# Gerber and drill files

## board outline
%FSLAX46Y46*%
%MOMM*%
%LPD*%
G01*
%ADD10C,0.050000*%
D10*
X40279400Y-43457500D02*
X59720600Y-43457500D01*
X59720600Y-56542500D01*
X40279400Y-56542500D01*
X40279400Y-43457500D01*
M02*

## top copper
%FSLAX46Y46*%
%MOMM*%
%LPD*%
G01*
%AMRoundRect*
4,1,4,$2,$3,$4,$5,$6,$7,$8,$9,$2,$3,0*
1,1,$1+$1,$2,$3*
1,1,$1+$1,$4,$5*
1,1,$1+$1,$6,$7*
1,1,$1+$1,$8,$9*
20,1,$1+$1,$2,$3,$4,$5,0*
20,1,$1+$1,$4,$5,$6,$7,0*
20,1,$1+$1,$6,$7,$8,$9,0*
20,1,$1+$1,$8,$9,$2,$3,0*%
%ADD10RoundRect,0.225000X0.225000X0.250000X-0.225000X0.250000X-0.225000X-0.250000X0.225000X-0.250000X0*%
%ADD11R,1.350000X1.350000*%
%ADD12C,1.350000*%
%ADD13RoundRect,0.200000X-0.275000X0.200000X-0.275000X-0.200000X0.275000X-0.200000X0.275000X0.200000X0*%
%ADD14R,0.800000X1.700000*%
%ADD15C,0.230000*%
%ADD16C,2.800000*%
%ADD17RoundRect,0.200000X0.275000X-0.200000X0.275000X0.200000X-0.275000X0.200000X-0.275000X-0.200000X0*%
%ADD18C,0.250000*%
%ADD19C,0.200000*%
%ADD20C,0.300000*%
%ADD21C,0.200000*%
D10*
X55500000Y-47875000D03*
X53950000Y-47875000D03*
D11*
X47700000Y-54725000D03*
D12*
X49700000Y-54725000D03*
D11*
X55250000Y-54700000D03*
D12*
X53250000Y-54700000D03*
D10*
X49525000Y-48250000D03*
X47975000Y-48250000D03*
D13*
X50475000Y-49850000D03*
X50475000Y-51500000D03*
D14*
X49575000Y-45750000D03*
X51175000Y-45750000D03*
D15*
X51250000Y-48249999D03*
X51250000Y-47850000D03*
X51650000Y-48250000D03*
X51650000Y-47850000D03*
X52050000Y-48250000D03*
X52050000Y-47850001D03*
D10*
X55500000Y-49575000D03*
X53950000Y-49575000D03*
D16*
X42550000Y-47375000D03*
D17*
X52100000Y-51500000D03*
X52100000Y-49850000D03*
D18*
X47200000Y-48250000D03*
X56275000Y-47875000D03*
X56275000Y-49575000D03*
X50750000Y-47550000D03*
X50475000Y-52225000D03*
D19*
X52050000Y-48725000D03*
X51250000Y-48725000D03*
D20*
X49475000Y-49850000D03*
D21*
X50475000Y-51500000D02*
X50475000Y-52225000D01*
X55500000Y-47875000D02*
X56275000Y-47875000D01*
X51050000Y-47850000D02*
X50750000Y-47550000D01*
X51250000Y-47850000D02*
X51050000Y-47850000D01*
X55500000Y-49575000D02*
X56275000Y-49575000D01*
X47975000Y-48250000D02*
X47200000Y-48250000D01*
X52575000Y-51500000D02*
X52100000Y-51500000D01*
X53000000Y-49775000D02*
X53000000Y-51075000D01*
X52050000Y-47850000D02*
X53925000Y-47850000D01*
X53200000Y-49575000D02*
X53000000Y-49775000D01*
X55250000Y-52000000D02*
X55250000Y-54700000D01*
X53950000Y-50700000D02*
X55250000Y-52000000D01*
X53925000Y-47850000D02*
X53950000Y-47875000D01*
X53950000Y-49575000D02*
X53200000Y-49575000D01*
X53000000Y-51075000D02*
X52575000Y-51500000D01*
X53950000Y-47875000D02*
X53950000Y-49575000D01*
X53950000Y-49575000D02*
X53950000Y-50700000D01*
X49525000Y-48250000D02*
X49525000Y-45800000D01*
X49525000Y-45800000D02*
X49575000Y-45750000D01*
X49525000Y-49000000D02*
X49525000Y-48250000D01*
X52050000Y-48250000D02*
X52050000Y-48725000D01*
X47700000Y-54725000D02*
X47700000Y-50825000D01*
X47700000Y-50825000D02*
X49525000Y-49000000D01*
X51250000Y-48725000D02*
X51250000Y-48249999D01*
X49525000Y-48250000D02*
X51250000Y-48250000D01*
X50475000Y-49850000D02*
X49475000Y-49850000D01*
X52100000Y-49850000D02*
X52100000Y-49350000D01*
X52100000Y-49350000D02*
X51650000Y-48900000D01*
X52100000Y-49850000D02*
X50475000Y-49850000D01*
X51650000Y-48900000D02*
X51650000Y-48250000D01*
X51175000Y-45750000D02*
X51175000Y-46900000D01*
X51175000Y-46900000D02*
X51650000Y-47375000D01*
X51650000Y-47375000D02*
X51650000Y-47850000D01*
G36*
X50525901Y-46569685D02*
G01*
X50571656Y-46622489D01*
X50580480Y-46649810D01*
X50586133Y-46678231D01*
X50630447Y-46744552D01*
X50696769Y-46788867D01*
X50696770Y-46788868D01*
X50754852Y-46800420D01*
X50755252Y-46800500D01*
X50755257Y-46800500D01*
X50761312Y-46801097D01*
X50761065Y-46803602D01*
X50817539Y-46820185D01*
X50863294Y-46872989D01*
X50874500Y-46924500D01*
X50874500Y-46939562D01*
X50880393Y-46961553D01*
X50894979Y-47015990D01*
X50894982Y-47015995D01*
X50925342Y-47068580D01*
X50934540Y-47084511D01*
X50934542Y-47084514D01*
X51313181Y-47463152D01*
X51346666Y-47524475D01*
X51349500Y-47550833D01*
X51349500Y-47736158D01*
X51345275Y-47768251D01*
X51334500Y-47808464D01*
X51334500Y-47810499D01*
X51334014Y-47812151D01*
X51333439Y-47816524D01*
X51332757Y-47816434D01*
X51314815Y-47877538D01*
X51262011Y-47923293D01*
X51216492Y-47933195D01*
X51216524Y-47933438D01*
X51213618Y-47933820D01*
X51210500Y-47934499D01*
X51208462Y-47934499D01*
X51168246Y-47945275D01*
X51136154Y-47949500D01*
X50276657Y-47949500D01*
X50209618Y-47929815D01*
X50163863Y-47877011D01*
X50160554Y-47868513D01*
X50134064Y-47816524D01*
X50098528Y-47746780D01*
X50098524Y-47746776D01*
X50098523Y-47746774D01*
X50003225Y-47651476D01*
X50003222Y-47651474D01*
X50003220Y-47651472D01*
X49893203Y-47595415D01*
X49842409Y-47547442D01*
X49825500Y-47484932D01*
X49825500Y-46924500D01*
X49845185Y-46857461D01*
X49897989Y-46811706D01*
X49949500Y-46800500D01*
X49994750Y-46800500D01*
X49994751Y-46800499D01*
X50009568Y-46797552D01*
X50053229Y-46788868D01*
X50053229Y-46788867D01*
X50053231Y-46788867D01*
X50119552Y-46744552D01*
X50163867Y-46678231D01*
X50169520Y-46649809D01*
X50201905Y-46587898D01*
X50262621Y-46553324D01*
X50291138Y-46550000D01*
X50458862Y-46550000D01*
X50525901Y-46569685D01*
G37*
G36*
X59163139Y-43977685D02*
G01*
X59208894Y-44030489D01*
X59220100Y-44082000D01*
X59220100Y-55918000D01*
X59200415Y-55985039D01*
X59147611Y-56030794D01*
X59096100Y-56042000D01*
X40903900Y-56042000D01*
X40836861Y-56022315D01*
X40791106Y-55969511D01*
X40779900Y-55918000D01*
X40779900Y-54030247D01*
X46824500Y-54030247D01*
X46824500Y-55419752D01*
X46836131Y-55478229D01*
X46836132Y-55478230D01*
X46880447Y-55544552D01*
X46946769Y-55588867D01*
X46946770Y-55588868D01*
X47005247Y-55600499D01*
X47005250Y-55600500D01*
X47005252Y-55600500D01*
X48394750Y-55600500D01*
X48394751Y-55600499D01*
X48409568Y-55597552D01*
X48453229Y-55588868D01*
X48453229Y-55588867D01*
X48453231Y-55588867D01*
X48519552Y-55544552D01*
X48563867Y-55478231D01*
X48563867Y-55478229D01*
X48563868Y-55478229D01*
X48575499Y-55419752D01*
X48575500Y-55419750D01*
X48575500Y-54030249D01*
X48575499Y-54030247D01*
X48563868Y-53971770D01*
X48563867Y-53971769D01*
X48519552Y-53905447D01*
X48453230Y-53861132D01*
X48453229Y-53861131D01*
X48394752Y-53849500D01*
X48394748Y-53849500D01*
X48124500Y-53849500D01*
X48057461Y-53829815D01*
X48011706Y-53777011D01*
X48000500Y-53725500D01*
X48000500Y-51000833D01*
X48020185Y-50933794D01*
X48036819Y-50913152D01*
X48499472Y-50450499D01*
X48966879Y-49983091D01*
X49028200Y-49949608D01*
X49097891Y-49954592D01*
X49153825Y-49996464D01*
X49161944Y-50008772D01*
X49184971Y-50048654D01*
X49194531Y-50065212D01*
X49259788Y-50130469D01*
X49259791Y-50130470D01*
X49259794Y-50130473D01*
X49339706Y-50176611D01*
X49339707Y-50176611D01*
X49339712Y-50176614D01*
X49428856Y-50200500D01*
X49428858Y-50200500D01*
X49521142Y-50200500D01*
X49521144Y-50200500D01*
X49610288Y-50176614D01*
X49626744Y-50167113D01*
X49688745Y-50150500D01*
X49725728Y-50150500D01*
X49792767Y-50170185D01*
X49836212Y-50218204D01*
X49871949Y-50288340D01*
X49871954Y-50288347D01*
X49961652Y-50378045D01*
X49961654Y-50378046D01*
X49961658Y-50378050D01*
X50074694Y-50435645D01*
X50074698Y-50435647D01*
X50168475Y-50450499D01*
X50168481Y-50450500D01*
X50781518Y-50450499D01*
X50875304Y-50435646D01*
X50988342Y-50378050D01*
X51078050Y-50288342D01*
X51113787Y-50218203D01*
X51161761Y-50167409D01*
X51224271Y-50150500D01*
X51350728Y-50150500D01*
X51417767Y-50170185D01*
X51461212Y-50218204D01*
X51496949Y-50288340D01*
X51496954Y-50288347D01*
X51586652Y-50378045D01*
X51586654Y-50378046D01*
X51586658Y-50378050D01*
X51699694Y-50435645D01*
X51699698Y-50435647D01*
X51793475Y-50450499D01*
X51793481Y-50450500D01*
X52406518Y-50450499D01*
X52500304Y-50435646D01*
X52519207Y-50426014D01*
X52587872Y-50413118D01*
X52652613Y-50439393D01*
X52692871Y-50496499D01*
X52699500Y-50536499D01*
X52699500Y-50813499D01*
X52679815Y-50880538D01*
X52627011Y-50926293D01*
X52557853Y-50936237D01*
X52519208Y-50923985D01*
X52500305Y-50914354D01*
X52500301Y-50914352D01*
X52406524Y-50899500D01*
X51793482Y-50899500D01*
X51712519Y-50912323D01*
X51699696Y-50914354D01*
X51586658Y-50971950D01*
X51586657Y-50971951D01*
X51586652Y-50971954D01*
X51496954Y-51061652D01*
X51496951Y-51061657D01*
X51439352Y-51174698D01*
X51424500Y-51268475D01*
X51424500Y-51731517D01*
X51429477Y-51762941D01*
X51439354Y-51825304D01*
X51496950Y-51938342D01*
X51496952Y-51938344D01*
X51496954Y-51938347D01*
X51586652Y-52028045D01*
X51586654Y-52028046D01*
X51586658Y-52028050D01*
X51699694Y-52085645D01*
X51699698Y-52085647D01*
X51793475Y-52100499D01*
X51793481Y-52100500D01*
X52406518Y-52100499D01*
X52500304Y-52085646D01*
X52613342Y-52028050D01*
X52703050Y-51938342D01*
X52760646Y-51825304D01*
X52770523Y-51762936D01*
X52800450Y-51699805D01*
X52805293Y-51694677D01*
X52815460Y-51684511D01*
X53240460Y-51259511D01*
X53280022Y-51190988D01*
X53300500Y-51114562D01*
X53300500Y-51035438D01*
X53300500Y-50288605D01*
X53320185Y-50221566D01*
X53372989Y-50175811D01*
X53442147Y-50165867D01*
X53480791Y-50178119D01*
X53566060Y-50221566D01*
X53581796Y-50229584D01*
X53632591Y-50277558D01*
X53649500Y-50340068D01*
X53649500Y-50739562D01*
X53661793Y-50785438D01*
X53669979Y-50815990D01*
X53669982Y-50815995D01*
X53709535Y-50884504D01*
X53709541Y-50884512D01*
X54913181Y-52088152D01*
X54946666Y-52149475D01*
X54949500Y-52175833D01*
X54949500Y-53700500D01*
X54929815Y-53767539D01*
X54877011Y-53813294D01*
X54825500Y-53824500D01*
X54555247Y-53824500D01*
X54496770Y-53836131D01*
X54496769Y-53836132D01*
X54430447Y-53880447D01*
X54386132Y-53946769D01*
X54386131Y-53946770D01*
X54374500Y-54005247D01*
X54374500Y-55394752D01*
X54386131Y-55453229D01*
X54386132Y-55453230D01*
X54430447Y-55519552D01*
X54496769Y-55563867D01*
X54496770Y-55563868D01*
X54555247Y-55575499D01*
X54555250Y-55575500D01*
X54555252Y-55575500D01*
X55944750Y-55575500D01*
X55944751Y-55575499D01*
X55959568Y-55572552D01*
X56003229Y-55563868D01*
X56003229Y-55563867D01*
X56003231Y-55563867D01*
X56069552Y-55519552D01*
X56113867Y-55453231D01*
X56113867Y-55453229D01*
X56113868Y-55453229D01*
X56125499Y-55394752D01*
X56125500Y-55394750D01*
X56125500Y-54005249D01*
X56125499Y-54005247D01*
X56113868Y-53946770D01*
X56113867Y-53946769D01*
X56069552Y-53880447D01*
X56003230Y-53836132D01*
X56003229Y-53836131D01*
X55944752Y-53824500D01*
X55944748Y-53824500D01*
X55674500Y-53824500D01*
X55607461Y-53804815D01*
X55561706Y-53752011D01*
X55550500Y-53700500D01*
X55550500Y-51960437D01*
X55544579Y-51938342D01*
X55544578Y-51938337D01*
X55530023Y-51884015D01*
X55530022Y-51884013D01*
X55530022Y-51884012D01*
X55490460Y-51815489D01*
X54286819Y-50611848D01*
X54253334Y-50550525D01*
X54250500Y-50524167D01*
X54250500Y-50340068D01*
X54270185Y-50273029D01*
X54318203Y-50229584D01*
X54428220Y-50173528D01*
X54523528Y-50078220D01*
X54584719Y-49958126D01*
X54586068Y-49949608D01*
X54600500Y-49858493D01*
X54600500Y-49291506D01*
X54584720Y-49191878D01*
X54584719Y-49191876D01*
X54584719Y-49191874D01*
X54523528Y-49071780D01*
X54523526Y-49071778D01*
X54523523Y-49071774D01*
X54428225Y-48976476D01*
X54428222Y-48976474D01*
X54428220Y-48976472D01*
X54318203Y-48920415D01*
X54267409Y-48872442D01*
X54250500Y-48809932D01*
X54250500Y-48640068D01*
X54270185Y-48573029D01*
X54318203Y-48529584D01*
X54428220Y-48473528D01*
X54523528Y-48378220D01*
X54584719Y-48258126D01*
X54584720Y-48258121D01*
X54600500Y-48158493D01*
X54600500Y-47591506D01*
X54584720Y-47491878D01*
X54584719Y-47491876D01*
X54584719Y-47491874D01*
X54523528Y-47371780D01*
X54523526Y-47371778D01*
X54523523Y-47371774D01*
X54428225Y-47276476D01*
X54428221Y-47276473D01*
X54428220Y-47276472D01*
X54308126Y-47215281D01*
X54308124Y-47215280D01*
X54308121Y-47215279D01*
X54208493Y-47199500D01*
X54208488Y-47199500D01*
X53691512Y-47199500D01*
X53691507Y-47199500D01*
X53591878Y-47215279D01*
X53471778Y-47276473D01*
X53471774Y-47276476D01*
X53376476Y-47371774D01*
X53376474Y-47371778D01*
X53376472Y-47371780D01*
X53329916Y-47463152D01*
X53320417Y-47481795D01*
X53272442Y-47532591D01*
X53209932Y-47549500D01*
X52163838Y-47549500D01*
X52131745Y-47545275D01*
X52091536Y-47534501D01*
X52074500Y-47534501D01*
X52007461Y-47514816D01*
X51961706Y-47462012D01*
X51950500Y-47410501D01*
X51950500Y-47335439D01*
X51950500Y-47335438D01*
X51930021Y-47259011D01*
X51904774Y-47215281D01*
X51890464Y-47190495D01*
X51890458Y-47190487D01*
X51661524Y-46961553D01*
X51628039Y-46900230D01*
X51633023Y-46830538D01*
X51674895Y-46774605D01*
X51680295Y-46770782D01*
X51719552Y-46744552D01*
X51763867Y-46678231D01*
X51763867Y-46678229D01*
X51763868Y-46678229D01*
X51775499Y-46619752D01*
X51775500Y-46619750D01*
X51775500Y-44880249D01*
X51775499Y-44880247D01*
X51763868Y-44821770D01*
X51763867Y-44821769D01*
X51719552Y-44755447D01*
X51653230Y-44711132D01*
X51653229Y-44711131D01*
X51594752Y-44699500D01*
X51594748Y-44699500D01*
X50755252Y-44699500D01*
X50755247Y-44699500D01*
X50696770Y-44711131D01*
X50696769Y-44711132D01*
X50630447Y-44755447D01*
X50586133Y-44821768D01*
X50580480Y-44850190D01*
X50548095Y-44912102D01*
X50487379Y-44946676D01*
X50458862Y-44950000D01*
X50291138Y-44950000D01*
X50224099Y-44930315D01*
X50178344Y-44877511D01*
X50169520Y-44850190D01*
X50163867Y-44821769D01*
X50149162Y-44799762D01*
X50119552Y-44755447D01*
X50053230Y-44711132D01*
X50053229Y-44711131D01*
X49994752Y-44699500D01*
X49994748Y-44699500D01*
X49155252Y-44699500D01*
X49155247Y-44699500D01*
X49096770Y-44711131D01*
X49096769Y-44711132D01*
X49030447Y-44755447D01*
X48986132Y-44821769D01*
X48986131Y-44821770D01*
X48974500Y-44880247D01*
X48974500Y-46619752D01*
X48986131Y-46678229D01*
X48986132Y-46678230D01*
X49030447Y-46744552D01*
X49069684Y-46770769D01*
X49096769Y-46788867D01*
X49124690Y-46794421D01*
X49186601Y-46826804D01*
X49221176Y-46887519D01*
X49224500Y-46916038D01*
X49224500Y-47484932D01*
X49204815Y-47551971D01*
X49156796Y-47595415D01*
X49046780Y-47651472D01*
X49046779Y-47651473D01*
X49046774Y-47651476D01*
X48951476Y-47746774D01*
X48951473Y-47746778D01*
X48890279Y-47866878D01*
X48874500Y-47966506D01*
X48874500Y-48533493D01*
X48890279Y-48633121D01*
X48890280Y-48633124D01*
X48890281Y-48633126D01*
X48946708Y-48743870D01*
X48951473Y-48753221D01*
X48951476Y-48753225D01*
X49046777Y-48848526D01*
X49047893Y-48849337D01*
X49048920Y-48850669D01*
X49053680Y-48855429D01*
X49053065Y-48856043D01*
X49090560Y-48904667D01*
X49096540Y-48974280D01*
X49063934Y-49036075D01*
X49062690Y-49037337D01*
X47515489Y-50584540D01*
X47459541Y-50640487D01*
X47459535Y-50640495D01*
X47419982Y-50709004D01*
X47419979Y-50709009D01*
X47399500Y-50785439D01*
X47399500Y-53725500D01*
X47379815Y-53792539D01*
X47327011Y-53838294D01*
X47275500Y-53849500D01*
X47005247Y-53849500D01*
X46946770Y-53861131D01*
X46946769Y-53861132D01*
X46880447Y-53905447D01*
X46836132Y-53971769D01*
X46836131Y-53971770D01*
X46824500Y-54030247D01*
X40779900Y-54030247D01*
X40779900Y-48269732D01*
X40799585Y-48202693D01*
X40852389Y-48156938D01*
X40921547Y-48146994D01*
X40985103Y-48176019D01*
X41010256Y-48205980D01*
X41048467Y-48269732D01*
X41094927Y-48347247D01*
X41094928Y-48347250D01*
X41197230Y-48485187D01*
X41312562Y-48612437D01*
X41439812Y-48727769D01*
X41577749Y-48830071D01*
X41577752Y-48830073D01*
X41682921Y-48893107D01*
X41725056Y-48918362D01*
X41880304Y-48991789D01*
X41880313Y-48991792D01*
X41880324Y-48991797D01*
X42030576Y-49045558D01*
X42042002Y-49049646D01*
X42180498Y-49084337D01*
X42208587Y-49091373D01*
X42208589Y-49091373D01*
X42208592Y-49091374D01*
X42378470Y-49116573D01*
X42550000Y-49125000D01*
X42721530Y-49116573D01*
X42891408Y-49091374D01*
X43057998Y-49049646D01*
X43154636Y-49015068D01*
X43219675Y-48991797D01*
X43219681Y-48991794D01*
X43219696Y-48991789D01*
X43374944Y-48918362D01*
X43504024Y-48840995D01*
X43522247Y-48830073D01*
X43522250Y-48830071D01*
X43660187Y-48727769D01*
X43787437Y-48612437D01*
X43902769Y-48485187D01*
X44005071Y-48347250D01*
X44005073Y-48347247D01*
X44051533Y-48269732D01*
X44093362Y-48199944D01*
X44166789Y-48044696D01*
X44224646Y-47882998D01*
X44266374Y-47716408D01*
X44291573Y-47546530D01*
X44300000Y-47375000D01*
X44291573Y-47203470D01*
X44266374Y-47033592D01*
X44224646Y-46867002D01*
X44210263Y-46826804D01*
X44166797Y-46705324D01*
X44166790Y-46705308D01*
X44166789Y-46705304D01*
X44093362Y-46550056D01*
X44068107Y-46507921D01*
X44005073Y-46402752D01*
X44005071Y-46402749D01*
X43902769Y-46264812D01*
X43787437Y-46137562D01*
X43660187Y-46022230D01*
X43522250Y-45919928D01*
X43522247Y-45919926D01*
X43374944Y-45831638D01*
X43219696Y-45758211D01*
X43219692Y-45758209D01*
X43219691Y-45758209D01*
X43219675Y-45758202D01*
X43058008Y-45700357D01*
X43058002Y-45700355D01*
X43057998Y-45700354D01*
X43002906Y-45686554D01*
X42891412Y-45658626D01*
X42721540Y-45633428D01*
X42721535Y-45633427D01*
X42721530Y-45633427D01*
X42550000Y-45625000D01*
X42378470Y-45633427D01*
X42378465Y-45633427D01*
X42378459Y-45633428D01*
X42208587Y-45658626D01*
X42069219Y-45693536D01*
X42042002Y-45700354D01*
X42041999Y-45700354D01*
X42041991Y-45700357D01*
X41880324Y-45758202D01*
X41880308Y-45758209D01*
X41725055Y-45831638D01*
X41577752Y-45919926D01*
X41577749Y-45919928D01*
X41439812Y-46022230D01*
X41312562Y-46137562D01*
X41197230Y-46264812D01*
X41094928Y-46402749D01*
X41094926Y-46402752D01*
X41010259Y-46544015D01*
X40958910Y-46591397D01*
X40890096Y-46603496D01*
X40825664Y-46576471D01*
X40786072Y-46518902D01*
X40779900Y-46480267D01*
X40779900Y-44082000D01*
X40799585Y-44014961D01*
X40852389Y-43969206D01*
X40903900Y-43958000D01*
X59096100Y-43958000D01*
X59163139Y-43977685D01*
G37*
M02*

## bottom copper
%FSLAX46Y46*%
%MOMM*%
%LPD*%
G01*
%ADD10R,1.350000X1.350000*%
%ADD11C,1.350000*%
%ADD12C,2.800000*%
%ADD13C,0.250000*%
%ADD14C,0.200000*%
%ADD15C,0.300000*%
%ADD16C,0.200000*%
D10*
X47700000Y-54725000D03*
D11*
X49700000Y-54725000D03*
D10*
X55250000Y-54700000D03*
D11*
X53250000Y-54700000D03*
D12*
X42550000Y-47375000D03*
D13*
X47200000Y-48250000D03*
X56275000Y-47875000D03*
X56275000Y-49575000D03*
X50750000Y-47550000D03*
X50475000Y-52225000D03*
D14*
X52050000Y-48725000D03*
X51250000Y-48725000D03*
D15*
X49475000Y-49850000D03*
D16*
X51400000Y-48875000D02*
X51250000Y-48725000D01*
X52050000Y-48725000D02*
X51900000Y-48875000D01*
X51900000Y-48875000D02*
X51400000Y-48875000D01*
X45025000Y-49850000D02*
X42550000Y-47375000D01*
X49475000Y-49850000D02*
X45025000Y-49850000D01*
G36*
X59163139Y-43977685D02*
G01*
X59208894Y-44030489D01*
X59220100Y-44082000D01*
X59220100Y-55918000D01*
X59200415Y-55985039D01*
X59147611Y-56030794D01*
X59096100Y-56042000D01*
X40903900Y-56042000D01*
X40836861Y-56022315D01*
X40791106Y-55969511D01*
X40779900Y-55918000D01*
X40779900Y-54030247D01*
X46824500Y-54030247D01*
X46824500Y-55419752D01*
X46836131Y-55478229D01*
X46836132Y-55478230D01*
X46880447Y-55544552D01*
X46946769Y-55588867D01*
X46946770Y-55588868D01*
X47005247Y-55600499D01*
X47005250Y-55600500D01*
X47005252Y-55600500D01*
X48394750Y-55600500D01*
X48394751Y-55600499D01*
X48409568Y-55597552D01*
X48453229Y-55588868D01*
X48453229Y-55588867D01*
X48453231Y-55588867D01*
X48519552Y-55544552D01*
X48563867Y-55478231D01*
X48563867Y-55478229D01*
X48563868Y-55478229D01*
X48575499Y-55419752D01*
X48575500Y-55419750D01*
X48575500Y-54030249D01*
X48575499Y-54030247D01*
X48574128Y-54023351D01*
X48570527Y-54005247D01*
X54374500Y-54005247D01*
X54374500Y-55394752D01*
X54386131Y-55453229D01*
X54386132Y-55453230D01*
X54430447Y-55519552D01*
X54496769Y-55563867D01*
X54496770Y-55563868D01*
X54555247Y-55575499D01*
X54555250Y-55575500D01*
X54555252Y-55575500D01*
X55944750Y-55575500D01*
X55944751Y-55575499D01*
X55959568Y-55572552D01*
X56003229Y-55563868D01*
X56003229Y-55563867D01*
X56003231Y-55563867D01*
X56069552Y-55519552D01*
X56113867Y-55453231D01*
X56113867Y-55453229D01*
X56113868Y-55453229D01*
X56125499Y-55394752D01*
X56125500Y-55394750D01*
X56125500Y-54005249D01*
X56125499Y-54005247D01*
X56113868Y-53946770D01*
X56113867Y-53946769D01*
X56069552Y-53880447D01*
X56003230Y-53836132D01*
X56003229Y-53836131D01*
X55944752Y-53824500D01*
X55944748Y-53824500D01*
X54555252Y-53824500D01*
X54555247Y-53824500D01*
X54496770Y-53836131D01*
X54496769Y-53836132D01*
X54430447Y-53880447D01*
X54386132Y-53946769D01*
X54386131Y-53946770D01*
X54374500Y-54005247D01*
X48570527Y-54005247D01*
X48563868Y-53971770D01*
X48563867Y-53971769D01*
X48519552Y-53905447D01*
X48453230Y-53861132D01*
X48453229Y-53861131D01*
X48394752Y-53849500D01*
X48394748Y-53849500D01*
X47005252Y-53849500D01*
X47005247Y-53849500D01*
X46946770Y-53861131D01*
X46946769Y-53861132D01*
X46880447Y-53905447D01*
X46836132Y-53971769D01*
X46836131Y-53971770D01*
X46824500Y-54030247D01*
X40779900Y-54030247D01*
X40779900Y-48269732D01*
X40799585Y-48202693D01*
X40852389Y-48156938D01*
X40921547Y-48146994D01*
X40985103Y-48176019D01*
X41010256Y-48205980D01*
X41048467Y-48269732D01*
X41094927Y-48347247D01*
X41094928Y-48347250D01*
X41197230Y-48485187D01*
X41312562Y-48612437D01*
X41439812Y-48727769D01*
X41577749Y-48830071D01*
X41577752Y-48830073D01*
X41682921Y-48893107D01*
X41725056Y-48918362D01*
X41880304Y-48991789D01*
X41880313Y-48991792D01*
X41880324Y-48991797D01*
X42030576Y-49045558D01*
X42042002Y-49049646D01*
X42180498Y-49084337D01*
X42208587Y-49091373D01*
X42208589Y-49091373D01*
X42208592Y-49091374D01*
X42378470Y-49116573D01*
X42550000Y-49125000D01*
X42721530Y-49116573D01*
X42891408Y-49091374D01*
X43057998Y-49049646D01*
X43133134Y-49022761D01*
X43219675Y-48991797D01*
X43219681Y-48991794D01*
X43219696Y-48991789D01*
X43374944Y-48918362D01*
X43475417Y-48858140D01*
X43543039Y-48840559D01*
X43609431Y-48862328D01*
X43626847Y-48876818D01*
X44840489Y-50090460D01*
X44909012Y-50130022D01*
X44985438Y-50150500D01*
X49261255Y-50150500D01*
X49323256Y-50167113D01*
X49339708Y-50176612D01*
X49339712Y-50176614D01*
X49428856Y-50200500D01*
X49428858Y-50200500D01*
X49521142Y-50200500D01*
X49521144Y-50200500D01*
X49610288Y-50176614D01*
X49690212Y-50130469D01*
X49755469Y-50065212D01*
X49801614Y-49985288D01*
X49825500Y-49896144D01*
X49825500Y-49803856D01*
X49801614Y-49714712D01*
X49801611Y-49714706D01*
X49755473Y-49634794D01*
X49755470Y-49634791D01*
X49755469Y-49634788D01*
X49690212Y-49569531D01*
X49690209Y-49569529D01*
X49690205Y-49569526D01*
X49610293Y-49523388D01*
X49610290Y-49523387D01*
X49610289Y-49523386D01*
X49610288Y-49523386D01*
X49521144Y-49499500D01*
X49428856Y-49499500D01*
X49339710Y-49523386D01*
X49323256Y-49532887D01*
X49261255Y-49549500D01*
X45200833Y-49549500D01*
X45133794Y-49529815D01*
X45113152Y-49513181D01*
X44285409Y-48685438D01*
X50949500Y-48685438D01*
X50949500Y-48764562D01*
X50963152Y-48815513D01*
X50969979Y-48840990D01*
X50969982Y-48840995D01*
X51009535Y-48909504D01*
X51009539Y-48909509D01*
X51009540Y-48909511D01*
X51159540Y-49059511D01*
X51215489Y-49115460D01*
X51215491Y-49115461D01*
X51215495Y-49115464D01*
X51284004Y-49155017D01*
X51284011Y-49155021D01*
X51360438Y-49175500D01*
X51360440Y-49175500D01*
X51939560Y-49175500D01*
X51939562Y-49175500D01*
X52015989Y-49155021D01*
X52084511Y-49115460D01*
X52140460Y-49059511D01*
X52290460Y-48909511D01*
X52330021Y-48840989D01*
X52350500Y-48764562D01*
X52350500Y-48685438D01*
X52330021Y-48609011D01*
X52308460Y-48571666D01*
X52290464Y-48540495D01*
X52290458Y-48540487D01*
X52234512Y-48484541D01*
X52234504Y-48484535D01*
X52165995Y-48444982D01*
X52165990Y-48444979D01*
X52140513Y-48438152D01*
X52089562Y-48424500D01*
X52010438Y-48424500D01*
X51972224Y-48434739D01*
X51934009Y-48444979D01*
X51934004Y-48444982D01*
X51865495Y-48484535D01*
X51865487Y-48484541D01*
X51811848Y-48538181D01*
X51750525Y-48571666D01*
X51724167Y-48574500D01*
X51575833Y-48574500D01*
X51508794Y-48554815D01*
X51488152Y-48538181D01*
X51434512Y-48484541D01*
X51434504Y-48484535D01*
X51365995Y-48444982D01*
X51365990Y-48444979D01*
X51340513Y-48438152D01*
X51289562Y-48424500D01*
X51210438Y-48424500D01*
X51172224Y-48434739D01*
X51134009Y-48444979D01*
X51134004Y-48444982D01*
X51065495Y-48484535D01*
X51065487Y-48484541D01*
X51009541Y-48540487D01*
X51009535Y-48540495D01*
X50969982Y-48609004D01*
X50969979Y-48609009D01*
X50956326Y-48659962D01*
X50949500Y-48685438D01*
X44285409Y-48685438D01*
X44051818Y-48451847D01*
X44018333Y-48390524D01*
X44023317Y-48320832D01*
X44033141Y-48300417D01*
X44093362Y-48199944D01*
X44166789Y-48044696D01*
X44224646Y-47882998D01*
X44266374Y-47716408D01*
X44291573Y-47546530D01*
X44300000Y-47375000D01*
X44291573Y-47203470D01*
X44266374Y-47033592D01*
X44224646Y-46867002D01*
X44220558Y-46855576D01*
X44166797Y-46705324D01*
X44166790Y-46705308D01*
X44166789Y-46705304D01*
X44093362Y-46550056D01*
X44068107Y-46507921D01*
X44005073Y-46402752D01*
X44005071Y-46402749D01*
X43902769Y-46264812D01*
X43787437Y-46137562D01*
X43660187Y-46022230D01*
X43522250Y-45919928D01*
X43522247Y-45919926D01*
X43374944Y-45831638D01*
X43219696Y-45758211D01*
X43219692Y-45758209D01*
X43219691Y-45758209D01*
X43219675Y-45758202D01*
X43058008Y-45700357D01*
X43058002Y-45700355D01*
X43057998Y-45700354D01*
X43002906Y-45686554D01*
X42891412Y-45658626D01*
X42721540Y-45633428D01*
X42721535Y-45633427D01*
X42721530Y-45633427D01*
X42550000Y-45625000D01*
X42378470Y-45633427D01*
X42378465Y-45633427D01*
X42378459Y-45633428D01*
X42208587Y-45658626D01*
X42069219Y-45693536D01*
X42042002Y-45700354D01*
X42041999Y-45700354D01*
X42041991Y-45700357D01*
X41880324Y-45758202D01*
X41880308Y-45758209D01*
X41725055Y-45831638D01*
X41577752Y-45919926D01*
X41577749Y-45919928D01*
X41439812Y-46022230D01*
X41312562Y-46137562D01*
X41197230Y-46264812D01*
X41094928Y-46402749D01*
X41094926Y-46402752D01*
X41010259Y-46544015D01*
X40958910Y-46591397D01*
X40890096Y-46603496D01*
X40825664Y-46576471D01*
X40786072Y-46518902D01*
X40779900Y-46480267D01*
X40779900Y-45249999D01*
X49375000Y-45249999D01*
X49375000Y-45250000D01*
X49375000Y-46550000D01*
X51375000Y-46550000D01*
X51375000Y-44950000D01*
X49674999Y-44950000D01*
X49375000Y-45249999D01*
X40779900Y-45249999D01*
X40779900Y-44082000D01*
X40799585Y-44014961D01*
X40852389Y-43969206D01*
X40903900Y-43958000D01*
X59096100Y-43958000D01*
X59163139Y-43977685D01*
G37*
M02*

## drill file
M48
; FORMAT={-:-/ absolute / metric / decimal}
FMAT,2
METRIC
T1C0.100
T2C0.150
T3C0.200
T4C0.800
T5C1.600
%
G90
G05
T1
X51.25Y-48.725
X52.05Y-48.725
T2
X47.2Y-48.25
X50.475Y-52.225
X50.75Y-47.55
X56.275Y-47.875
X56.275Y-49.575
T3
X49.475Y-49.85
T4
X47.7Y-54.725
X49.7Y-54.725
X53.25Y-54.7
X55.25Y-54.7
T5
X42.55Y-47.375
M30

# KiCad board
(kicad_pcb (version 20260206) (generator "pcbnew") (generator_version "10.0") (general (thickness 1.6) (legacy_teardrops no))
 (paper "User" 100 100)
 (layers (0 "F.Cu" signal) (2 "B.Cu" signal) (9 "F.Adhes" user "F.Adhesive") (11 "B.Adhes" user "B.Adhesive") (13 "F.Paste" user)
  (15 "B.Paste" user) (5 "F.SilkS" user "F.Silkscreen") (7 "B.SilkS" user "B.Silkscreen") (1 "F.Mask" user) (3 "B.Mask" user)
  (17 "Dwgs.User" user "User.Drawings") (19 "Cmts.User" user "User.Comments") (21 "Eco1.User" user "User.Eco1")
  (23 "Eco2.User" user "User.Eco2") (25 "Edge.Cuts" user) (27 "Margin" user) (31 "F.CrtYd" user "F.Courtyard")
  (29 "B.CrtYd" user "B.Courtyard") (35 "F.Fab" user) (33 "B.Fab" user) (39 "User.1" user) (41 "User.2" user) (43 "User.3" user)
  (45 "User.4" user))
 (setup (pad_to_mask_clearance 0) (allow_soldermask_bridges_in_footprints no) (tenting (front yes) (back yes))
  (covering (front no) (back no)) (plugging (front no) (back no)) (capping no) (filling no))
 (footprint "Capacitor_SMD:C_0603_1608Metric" (layer "F.Cu") (at 54.725 47.875 180)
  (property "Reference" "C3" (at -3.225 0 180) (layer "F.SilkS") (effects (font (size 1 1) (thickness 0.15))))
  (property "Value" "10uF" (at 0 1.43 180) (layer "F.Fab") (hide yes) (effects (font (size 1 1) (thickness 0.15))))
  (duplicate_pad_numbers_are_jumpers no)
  (pad "1" smd roundrect (at -0.775 0 180) (size 0.9 0.95) (layers "F.Cu" "F.Mask" "F.Paste") (roundrect_rratio 0.25) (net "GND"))
  (pad "2" smd roundrect (at 0.775 0 180) (size 0.9 0.95) (layers "F.Cu" "F.Mask" "F.Paste") (roundrect_rratio 0.25) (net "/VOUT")))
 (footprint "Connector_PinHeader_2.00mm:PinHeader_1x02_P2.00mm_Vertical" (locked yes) (layer "F.Cu") (at 48.7 54.725 90)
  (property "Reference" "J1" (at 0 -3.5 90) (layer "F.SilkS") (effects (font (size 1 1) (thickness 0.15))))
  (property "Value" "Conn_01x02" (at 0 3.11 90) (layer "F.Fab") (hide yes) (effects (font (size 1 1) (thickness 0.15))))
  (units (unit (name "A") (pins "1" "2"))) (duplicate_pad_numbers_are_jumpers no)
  (pad "1" thru_hole rect (at 0 -1 90) (size 1.35 1.35) (drill 0.8) (layers "*.Cu" "*.Mask") (remove_unused_layers no) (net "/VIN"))
  (pad "2" thru_hole circle (at 0 1 90) (size 1.35 1.35) (drill 0.8) (layers "*.Cu" "*.Mask") (remove_unused_layers no) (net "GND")))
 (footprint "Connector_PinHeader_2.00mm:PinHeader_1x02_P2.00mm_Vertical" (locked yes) (layer "F.Cu") (at 54.25 54.7 -90)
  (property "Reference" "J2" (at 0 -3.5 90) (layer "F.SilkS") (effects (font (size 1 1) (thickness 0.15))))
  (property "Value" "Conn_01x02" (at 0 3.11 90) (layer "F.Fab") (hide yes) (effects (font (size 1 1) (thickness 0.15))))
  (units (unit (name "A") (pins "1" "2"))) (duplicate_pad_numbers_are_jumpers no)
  (pad "1" thru_hole rect (at 0 -1 270) (size 1.35 1.35) (drill 0.8) (layers "*.Cu" "*.Mask") (remove_unused_layers no) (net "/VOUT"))
  (pad "2" thru_hole circle (at 0 1 270) (size 1.35 1.35) (drill 0.8) (layers "*.Cu" "*.Mask") (remove_unused_layers no) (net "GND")))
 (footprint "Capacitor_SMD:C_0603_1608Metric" (layer "F.Cu") (at 48.75 48.25 180)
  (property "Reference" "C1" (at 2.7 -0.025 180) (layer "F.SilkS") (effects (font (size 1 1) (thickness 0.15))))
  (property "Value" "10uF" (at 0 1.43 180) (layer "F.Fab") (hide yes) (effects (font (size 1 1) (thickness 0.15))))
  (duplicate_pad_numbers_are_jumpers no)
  (pad "1" smd roundrect (at -0.775 0 180) (size 0.9 0.95) (layers "F.Cu" "F.Mask" "F.Paste") (roundrect_rratio 0.25) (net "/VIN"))
  (pad "2" smd roundrect (at 0.775 0 180) (size 0.9 0.95) (layers "F.Cu" "F.Mask" "F.Paste") (roundrect_rratio 0.25) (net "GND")))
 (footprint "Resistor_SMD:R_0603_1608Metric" (layer "F.Cu") (at 50.475 50.675 -90)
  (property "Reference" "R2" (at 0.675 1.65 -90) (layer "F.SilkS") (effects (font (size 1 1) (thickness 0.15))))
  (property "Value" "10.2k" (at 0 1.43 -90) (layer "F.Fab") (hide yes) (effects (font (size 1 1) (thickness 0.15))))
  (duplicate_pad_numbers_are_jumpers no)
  (pad "1" smd roundrect (at -0.825 0 -90) (size 0.8 0.95) (layers "F.Cu" "F.Mask" "F.Paste") (roundrect_rratio 0.25) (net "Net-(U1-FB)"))
  (pad "2" smd roundrect (at 0.825 0 -90) (size 0.8 0.95) (layers "F.Cu" "F.Mask" "F.Paste") (roundrect_rratio 0.25) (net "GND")))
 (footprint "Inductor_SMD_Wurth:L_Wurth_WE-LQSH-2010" (layer "F.Cu") (at 50.375 45.75)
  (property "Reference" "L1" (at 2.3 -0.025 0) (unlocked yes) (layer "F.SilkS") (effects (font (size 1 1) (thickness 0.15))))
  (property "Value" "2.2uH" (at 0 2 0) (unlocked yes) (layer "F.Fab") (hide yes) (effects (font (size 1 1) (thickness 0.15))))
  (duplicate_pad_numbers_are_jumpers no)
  (pad "1" smd rect (at -0.8 0) (size 0.8 1.7) (layers "F.Cu" "F.Mask" "F.Paste") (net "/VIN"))
  (pad "2" smd rect (at 0.8 0) (size 0.8 1.7) (layers "F.Cu" "F.Mask" "F.Paste") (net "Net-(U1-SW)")))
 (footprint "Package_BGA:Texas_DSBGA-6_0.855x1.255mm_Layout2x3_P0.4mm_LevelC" (layer "F.Cu") (at 51.65 48.05 90)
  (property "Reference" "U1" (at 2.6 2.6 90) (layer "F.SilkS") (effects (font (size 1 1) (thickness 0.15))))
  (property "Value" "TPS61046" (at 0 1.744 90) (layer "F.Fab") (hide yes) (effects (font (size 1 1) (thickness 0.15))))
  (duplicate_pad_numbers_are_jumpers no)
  (pad "A1" smd circle (at -0.199999 -0.4 90) (size 0.23 0.23) (layers "F.Cu" "F.Mask") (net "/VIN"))
  (pad "A2" smd circle (at 0.2 -0.4 90) (size 0.23 0.23) (layers "F.Cu" "F.Mask") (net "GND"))
  (pad "B1" smd circle (at -0.2 0 90) (size 0.23 0.23) (layers "F.Cu" "F.Mask") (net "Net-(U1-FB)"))
  (pad "B2" smd circle (at 0.2 0 90) (size 0.23 0.23) (layers "F.Cu" "F.Mask") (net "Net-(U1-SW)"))
  (pad "C1" smd circle (at -0.2 0.4 90) (size 0.23 0.23) (layers "F.Cu" "F.Mask") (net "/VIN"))
  (pad "C2" smd circle (at 0.199999 0.4 90) (size 0.23 0.23) (layers "F.Cu" "F.Mask") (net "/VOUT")))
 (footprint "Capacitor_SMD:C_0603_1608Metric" (layer "F.Cu") (at 54.725 49.575 180)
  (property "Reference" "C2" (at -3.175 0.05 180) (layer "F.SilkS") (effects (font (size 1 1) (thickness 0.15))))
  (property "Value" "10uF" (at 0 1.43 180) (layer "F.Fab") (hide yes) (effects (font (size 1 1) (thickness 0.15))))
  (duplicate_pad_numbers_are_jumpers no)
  (pad "1" smd roundrect (at -0.775 0 180) (size 0.9 0.95) (layers "F.Cu" "F.Mask" "F.Paste") (roundrect_rratio 0.25) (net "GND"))
  (pad "2" smd roundrect (at 0.775 0 180) (size 0.9 0.95) (layers "F.Cu" "F.Mask" "F.Paste") (roundrect_rratio 0.25) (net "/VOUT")))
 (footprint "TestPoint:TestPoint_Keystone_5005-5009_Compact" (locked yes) (layer "F.Cu") (at 42.55 47.375)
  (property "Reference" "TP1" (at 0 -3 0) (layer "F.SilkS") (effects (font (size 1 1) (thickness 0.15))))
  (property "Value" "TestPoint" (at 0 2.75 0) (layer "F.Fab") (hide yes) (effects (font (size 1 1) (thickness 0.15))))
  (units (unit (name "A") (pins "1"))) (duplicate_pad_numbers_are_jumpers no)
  (pad "1" thru_hole circle (at 0 0) (size 2.8 2.8) (drill 1.6) (layers "*.Cu" "*.Mask") (remove_unused_layers no) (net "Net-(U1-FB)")))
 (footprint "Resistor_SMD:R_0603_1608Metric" (layer "F.Cu") (at 52.1 50.675 90)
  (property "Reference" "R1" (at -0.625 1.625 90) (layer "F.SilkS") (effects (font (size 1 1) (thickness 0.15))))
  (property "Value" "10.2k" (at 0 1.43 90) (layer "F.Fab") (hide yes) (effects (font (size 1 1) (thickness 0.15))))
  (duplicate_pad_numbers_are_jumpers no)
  (pad "1" smd roundrect (at -0.825 0 90) (size 0.8 0.95) (layers "F.Cu" "F.Mask" "F.Paste") (roundrect_rratio 0.25) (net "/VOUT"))
  (pad "2" smd roundrect (at 0.825 0 90) (size 0.8 0.95) (layers "F.Cu" "F.Mask" "F.Paste") (roundrect_rratio 0.25) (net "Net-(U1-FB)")))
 (gr_rect (start 40.2794 43.4575) (end 59.7206 56.5425) (stroke (width 0.05) (type solid)) (fill no) (locked yes) (layer "Edge.Cuts"))
 (segment (start 50.475 51.5) (end 50.475 52.225) (width 0.2) (layer "F.Cu") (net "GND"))
 (segment (start 55.5 47.875) (end 56.275 47.875) (width 0.2) (layer "F.Cu") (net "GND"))
 (segment (start 51.05 47.85) (end 50.75 47.55) (width 0.2) (layer "F.Cu") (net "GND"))
 (segment (start 51.25 47.85) (end 51.05 47.85) (width 0.2) (layer "F.Cu") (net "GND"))
 (segment (start 55.5 49.575) (end 56.275 49.575) (width 0.2) (layer "F.Cu") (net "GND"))
 (segment (start 47.975 48.25) (end 47.2 48.25) (width 0.2) (layer "F.Cu") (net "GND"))
 (via (at 47.2 48.25) (size 0.25) (drill 0.15) (layers "F.Cu" "B.Cu") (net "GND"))
 (via (at 56.275 47.875) (size 0.25) (drill 0.15) (layers "F.Cu" "B.Cu") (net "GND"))
 (via (at 56.275 49.575) (size 0.25) (drill 0.15) (layers "F.Cu" "B.Cu") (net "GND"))
 (via (at 50.75 47.55) (size 0.25) (drill 0.15) (layers "F.Cu" "B.Cu") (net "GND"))
 (via (at 50.475 52.225) (size 0.25) (drill 0.15) (layers "F.Cu" "B.Cu") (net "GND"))
 (segment (start 52.575 51.5) (end 52.1 51.5) (width 0.2) (layer "F.Cu") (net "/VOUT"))
 (segment (start 53 49.775) (end 53 51.075) (width 0.2) (layer "F.Cu") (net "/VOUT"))
 (segment (start 52.05 47.85) (end 53.925 47.85) (width 0.2) (layer "F.Cu") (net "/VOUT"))
 (segment (start 53.2 49.575) (end 53 49.775) (width 0.2) (layer "F.Cu") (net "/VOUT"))
 (segment (start 55.25 52) (end 55.25 54.7) (width 0.2) (layer "F.Cu") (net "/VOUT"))
 (segment (start 53.95 50.7) (end 55.25 52) (width 0.2) (layer "F.Cu") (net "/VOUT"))
 (segment (start 53.925 47.85) (end 53.95 47.875) (width 0.2) (layer "F.Cu") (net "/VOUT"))
 (segment (start 53.95 49.575) (end 53.2 49.575) (width 0.2) (layer "F.Cu") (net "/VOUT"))
 (segment (start 53 51.075) (end 52.575 51.5) (width 0.2) (layer "F.Cu") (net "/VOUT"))
 (segment (start 53.95 47.875) (end 53.95 49.575) (width 0.2) (layer "F.Cu") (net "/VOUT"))
 (segment (start 53.95 49.575) (end 53.95 50.7) (width 0.2) (layer "F.Cu") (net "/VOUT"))
 (segment (start 49.525 48.25) (end 49.525 45.8) (width 0.2) (layer "F.Cu") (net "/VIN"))
 (segment (start 49.525 45.8) (end 49.575 45.75) (width 0.2) (layer "F.Cu") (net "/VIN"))
 (segment (start 49.525 49) (end 49.525 48.25) (width 0.2) (layer "F.Cu") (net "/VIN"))
 (segment (start 52.05 48.25) (end 52.05 48.725) (width 0.2) (layer "F.Cu") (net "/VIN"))
 (segment (start 47.7 54.725) (end 47.7 50.825) (width 0.2) (layer "F.Cu") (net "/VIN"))
 (segment (start 47.7 50.825) (end 49.525 49) (width 0.2) (layer "F.Cu") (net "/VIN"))
 (segment (start 51.25 48.725) (end 51.25 48.249999) (width 0.2) (layer "F.Cu") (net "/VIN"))
 (segment (start 49.525 48.25) (end 51.25 48.25) (width 0.2) (layer "F.Cu") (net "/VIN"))
 (via (at 52.05 48.725) (size 0.2) (drill 0.1) (layers "F.Cu" "B.Cu") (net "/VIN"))
 (via (at 51.25 48.725) (size 0.2) (drill 0.1) (layers "F.Cu" "B.Cu") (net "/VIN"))
 (segment (start 51.4 48.875) (end 51.25 48.725) (width 0.2) (layer "B.Cu") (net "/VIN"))
 (segment (start 52.05 48.725) (end 51.9 48.875) (width 0.2) (layer "B.Cu") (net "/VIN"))
 (segment (start 51.9 48.875) (end 51.4 48.875) (width 0.2) (layer "B.Cu") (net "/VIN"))
 (segment (start 50.475 49.85) (end 49.475 49.85) (width 0.2) (layer "F.Cu") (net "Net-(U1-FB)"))
 (segment (start 52.1 49.85) (end 52.1 49.35) (width 0.2) (layer "F.Cu") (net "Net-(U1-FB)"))
 (segment (start 52.1 49.35) (end 51.65 48.9) (width 0.2) (layer "F.Cu") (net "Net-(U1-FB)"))
 (segment (start 52.1 49.85) (end 50.475 49.85) (width 0.2) (layer "F.Cu") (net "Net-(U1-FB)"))
 (segment (start 51.65 48.9) (end 51.65 48.25) (width 0.2) (layer "F.Cu") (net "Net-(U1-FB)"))
 (via (at 49.475 49.85) (size 0.3) (drill 0.2) (layers "F.Cu" "B.Cu") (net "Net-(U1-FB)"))
 (segment (start 45.025 49.85) (end 42.55 47.375) (width 0.2) (layer "B.Cu") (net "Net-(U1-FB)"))
 (segment (start 49.475 49.85) (end 45.025 49.85) (width 0.2) (layer "B.Cu") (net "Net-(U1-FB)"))
 (segment (start 51.175 45.75) (end 51.175 46.9) (width 0.2) (layer "F.Cu") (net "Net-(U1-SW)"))
 (segment (start 51.175 46.9) (end 51.65 47.375) (width 0.2) (layer "F.Cu") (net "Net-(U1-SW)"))
 (segment (start 51.65 47.375) (end 51.65 47.85) (width 0.2) (layer "F.Cu") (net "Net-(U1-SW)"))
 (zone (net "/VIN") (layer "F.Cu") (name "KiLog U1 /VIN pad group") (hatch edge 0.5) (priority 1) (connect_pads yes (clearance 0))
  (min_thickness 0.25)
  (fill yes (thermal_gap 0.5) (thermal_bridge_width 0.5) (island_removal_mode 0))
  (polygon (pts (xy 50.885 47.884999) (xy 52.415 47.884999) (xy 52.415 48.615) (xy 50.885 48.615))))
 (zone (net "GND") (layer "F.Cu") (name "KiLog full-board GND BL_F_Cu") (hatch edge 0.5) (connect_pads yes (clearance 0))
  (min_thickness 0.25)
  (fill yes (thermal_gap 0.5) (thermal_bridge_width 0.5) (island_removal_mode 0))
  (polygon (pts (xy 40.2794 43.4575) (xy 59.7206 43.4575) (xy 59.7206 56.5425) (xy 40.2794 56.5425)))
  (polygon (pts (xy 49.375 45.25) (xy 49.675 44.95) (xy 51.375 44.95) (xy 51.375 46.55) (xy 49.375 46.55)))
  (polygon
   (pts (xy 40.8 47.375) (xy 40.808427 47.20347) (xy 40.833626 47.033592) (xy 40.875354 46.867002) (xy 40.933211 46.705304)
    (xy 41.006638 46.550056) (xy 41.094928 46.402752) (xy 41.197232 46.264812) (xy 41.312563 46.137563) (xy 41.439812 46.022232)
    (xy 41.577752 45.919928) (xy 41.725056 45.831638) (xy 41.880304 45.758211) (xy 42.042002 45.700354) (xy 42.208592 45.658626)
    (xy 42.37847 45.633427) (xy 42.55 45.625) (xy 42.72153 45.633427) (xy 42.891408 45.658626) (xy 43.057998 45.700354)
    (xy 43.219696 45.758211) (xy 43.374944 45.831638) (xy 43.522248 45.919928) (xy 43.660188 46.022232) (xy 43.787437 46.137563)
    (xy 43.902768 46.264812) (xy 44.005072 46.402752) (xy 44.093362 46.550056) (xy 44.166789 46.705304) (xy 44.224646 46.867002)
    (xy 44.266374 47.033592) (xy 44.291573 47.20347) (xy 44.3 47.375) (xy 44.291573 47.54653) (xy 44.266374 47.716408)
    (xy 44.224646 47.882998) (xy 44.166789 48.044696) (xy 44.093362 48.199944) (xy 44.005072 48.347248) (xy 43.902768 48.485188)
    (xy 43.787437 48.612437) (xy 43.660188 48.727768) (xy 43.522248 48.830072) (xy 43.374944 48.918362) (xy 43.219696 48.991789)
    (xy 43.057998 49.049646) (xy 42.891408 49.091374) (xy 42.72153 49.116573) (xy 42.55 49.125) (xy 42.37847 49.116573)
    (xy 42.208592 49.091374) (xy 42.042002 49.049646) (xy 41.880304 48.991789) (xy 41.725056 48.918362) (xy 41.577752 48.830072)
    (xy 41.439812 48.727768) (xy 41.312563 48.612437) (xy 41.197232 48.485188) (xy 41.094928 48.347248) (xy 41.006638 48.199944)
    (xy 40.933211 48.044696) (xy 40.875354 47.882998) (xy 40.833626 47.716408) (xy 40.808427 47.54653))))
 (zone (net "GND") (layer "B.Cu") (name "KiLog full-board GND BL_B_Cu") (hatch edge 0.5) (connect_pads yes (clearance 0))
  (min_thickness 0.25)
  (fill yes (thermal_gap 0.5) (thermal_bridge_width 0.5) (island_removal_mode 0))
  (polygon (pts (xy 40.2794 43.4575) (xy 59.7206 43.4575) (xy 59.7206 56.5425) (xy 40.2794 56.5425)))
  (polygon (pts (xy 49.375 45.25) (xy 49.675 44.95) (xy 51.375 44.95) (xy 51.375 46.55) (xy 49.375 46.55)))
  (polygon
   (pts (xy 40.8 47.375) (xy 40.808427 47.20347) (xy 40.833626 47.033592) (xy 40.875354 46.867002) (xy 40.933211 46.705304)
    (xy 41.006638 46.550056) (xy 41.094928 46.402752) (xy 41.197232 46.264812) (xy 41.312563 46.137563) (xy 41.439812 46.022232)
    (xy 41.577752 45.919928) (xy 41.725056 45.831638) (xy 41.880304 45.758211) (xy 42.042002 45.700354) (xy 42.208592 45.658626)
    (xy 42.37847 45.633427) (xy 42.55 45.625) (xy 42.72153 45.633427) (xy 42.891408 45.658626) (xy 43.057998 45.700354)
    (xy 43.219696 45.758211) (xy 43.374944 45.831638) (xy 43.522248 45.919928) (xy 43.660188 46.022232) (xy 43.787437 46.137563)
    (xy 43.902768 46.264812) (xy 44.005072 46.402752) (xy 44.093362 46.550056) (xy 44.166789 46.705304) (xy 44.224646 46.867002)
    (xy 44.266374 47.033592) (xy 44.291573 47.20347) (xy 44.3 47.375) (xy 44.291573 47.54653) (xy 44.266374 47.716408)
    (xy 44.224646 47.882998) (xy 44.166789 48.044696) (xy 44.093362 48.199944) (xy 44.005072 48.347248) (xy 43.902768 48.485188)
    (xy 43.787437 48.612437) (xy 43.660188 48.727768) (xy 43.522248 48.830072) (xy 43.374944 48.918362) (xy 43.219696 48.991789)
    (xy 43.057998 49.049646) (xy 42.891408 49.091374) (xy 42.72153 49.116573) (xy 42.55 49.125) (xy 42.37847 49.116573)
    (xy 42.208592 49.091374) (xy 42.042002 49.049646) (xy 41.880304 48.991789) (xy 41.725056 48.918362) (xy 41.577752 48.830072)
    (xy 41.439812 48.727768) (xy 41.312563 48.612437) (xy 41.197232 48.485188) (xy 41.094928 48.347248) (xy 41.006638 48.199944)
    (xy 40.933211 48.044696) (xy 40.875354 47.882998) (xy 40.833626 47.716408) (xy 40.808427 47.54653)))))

